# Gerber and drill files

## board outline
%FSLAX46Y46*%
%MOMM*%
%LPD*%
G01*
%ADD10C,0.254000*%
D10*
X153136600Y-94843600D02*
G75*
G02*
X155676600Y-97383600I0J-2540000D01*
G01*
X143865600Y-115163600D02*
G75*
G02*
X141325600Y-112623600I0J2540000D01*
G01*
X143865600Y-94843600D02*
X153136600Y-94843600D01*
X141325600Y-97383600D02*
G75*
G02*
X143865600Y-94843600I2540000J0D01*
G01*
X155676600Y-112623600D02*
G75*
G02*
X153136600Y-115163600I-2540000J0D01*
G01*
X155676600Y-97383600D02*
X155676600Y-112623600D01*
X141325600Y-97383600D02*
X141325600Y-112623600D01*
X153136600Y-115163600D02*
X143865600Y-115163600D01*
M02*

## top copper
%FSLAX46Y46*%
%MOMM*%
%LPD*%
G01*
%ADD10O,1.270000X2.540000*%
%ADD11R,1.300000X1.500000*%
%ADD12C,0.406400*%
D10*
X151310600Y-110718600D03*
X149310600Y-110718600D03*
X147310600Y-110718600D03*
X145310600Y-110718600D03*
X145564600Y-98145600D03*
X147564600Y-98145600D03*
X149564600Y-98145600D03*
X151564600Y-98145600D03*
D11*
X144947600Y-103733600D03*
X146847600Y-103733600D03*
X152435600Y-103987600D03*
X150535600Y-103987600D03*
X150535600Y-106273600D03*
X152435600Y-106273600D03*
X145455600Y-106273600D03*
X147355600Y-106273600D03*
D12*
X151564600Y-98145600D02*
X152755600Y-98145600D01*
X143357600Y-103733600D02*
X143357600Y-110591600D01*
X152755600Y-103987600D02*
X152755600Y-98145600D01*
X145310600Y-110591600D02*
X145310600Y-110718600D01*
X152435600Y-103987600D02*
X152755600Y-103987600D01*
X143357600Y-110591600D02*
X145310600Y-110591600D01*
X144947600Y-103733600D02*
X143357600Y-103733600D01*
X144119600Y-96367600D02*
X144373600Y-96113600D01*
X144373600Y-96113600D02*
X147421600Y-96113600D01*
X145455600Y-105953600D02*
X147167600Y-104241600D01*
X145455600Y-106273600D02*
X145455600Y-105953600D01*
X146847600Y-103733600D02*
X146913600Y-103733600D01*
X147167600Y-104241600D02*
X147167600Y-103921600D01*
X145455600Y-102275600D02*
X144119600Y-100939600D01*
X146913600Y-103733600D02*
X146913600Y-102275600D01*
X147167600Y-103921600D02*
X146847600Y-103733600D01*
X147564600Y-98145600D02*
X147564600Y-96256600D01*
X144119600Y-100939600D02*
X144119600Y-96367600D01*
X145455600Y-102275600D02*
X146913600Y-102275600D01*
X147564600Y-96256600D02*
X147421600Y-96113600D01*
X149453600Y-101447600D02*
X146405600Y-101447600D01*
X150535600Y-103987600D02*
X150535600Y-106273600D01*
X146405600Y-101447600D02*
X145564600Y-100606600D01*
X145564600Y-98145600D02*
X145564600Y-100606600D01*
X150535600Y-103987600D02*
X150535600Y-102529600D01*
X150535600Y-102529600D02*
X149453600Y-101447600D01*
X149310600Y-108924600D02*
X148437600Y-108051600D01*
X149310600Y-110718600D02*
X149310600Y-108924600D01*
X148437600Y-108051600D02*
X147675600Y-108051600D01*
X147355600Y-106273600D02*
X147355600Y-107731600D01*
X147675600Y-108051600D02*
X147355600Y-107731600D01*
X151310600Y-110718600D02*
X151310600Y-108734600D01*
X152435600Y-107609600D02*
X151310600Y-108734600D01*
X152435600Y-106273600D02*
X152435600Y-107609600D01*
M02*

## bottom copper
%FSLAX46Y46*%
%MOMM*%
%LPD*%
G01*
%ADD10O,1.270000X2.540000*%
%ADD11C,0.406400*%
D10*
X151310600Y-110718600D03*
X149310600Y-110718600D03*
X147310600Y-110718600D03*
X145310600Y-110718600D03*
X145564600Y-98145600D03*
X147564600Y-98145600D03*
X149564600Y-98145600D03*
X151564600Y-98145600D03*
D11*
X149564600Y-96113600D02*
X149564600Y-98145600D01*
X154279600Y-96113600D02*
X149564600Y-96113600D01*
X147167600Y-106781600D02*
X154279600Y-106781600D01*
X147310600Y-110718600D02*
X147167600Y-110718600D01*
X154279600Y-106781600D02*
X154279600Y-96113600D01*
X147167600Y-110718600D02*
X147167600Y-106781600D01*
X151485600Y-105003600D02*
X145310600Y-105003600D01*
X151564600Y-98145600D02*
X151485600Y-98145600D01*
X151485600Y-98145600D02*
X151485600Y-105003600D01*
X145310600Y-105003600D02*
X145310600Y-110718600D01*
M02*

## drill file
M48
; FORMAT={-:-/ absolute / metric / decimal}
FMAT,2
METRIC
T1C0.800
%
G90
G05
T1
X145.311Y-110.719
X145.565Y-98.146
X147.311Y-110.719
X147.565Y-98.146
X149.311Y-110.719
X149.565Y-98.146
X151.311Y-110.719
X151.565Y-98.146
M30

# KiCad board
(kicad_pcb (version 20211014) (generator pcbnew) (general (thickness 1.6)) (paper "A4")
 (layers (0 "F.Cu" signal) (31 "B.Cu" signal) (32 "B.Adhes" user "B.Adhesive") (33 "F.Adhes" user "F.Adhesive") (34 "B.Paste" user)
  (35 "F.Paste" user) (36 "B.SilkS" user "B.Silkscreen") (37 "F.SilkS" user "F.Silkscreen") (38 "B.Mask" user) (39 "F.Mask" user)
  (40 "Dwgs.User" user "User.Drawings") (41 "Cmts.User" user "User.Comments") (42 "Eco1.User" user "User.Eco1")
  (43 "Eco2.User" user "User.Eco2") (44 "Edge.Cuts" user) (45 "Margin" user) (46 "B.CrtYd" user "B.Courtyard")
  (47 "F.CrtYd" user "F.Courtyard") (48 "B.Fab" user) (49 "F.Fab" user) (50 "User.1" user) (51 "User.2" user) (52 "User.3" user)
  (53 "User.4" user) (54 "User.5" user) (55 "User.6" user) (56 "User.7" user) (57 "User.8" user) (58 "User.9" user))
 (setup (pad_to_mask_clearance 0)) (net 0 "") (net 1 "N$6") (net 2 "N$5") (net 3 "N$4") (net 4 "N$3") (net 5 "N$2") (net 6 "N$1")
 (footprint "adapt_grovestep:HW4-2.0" (layer "F.Cu") (at 148.3106 110.7186 180)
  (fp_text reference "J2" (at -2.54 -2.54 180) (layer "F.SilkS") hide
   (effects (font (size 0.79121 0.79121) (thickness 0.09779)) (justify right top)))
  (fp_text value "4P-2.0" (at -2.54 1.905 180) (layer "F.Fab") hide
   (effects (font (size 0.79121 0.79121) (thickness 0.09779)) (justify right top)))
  (pad "1" thru_hole oval (at -3 0 270) (size 2.54 1.27) (drill 0.8) (layers *.Cu *.Mask) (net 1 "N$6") (solder_mask_margin 0.1016))
  (pad "2" thru_hole oval (at -1 0 270) (size 2.54 1.27) (drill 0.8) (layers *.Cu *.Mask) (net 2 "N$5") (solder_mask_margin 0.1016))
  (pad "3" thru_hole oval (at 1 0 270) (size 2.54 1.27) (drill 0.8) (layers *.Cu *.Mask) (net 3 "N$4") (solder_mask_margin 0.1016))
  (pad "4" thru_hole oval (at 3 0 270) (size 2.54 1.27) (drill 0.8) (layers *.Cu *.Mask) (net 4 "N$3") (solder_mask_margin 0.1016)))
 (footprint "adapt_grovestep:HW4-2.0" (layer "F.Cu") (at 148.5646 98.1456)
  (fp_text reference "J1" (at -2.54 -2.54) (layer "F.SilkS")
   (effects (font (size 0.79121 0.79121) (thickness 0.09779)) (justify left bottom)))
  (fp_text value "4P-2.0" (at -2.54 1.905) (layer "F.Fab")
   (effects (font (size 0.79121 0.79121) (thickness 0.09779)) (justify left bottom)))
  (pad "1" thru_hole oval (at -3 0 90) (size 2.54 1.27) (drill 0.8) (layers *.Cu *.Mask) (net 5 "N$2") (solder_mask_margin 0.1016))
  (pad "2" thru_hole oval (at -1 0 90) (size 2.54 1.27) (drill 0.8) (layers *.Cu *.Mask) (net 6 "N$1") (solder_mask_margin 0.1016))
  (pad "3" thru_hole oval (at 1 0 90) (size 2.54 1.27) (drill 0.8) (layers *.Cu *.Mask) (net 3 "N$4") (solder_mask_margin 0.1016))
  (pad "4" thru_hole oval (at 3 0 90) (size 2.54 1.27) (drill 0.8) (layers *.Cu *.Mask) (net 4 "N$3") (solder_mask_margin 0.1016)))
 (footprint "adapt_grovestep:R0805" (layer "F.Cu") (at 145.8976 103.7336)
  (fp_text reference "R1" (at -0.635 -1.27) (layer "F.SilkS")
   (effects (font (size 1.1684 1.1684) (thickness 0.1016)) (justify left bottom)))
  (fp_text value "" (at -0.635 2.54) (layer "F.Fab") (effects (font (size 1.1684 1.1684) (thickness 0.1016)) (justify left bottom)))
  (pad "1" smd rect (at -0.95 0) (size 1.3 1.5) (layers "F.Cu" "F.Paste" "F.Mask") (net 4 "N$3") (solder_mask_margin 0.1016))
  (pad "2" smd rect (at 0.95 0) (size 1.3 1.5) (layers "F.Cu" "F.Paste" "F.Mask") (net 6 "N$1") (solder_mask_margin 0.1016)))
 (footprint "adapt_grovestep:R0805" (layer "F.Cu") (at 151.4856 103.9876 180)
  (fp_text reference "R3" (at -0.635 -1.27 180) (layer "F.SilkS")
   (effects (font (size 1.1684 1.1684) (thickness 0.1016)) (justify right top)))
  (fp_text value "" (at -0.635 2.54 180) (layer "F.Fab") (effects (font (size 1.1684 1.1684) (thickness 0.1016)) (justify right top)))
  (pad "1" smd rect (at -0.95 0 180) (size 1.3 1.5) (layers "F.Cu" "F.Paste" "F.Mask") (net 4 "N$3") (solder_mask_margin 0.1016))
  (pad "2" smd rect (at 0.95 0 180) (size 1.3 1.5) (layers "F.Cu" "F.Paste" "F.Mask") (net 5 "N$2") (solder_mask_margin 0.1016)))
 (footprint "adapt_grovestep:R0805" (layer "F.Cu") (at 151.4856 106.2736)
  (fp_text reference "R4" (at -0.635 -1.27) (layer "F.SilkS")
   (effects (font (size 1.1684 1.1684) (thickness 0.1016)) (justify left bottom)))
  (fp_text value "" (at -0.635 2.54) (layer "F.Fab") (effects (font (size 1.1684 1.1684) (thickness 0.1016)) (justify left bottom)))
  (pad "1" smd rect (at -0.95 0) (size 1.3 1.5) (layers "F.Cu" "F.Paste" "F.Mask") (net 5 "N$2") (solder_mask_margin 0.1016))
  (pad "2" smd rect (at 0.95 0) (size 1.3 1.5) (layers "F.Cu" "F.Paste" "F.Mask") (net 1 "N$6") (solder_mask_margin 0.1016)))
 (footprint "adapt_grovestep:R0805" (layer "F.Cu") (at 146.4056 106.2736)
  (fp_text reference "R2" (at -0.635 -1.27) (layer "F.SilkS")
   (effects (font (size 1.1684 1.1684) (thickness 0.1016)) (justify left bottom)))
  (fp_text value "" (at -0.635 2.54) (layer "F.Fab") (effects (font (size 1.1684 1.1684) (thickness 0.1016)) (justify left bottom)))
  (pad "1" smd rect (at -0.95 0) (size 1.3 1.5) (layers "F.Cu" "F.Paste" "F.Mask") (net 6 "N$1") (solder_mask_margin 0.1016))
  (pad "2" smd rect (at 0.95 0) (size 1.3 1.5) (layers "F.Cu" "F.Paste" "F.Mask") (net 2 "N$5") (solder_mask_margin 0.1016)))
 (gr_arc (start 153.1366 94.8436) (mid 154.932651 95.587549) (end 155.6766 97.3836) (layer "Edge.Cuts") (width 0.254))
 (gr_arc (start 143.8656 115.1636) (mid 142.069549 114.419651) (end 141.3256 112.6236) (layer "Edge.Cuts") (width 0.254))
 (gr_line (start 143.8656 94.8436) (end 153.1366 94.8436) (layer "Edge.Cuts") (width 0.254))
 (gr_arc (start 141.3256 97.3836) (mid 142.069549 95.587549) (end 143.8656 94.8436) (layer "Edge.Cuts") (width 0.254))
 (gr_arc (start 155.6766 112.6236) (mid 154.932651 114.419651) (end 153.1366 115.1636) (layer "Edge.Cuts") (width 0.254))
 (gr_line (start 155.6766 97.3836) (end 155.6766 112.6236) (layer "Edge.Cuts") (width 0.254))
 (gr_line (start 141.3256 97.3836) (end 141.3256 112.6236) (layer "Edge.Cuts") (width 0.254))
 (gr_line (start 153.1366 115.1636) (end 143.8656 115.1636) (layer "Edge.Cuts") (width 0.254))
 (segment (start 149.5646 96.1136) (end 149.5646 98.1456) (width 0.4064) (layer "B.Cu") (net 3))
 (segment (start 154.2796 96.1136) (end 149.5646 96.1136) (width 0.4064) (layer "B.Cu") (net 3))
 (segment (start 147.1676 106.7816) (end 154.2796 106.7816) (width 0.4064) (layer "B.Cu") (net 3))
 (segment (start 147.3106 110.7186) (end 147.1676 110.7186) (width 0.4064) (layer "B.Cu") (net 3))
 (segment (start 154.2796 106.7816) (end 154.2796 96.1136) (width 0.4064) (layer "B.Cu") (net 3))
 (segment (start 147.1676 110.7186) (end 147.1676 106.7816) (width 0.4064) (layer "B.Cu") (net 3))
 (segment (start 151.5646 98.1456) (end 152.7556 98.1456) (width 0.4064) (layer "F.Cu") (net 4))
 (segment (start 143.3576 103.7336) (end 143.3576 110.5916) (width 0.4064) (layer "F.Cu") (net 4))
 (segment (start 152.7556 103.9876) (end 152.7556 98.1456) (width 0.4064) (layer "F.Cu") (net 4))
 (segment (start 145.3106 110.5916) (end 145.3106 110.7186) (width 0.4064) (layer "F.Cu") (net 4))
 (segment (start 152.4356 103.9876) (end 152.7556 103.9876) (width 0.4064) (layer "F.Cu") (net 4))
 (segment (start 143.3576 110.5916) (end 145.3106 110.5916) (width 0.4064) (layer "F.Cu") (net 4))
 (segment (start 144.9476 103.7336) (end 143.3576 103.7336) (width 0.4064) (layer "F.Cu") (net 4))
 (segment (start 151.4856 105.0036) (end 145.3106 105.0036) (width 0.4064) (layer "B.Cu") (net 4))
 (segment (start 151.5646 98.1456) (end 151.4856 98.1456) (width 0.4064) (layer "B.Cu") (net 4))
 (segment (start 151.4856 98.1456) (end 151.4856 105.0036) (width 0.4064) (layer "B.Cu") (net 4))
 (segment (start 145.3106 105.0036) (end 145.3106 110.7186) (width 0.4064) (layer "B.Cu") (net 4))
 (segment (start 144.1196 96.3676) (end 144.3736 96.1136) (width 0.4064) (layer "F.Cu") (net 6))
 (segment (start 144.3736 96.1136) (end 147.4216 96.1136) (width 0.4064) (layer "F.Cu") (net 6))
 (segment (start 145.4556 105.9536) (end 147.1676 104.2416) (width 0.4064) (layer "F.Cu") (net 6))
 (segment (start 145.4556 106.2736) (end 145.4556 105.9536) (width 0.4064) (layer "F.Cu") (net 6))
 (segment (start 146.8476 103.7336) (end 146.9136 103.7336) (width 0.4064) (layer "F.Cu") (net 6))
 (segment (start 147.1676 104.2416) (end 147.1676 103.9216) (width 0.4064) (layer "F.Cu") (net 6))
 (segment (start 145.4556 102.2756) (end 144.1196 100.9396) (width 0.4064) (layer "F.Cu") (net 6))
 (segment (start 146.9136 103.7336) (end 146.9136 102.2756) (width 0.4064) (layer "F.Cu") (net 6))
 (segment (start 147.1676 103.9216) (end 146.8476 103.7336) (width 0.4064) (layer "F.Cu") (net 6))
 (segment (start 147.5646 98.1456) (end 147.5646 96.2566) (width 0.4064) (layer "F.Cu") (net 6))
 (segment (start 144.1196 100.9396) (end 144.1196 96.3676) (width 0.4064) (layer "F.Cu") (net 6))
 (segment (start 145.4556 102.2756) (end 146.9136 102.2756) (width 0.4064) (layer "F.Cu") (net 6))
 (segment (start 147.5646 96.2566) (end 147.4216 96.1136) (width 0.4064) (layer "F.Cu") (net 6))
 (segment (start 149.4536 101.4476) (end 146.4056 101.4476) (width 0.4064) (layer "F.Cu") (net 5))
 (segment (start 150.5356 103.9876) (end 150.5356 106.2736) (width 0.4064) (layer "F.Cu") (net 5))
 (segment (start 146.4056 101.4476) (end 145.5646 100.6066) (width 0.4064) (layer "F.Cu") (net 5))
 (segment (start 145.5646 98.1456) (end 145.5646 100.6066) (width 0.4064) (layer "F.Cu") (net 5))
 (segment (start 150.5356 103.9876) (end 150.5356 102.5296) (width 0.4064) (layer "F.Cu") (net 5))
 (segment (start 150.5356 102.5296) (end 149.4536 101.4476) (width 0.4064) (layer "F.Cu") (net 5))
 (segment (start 149.3106 108.9246) (end 148.4376 108.0516) (width 0.4064) (layer "F.Cu") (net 2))
 (segment (start 149.3106 110.7186) (end 149.3106 108.9246) (width 0.4064) (layer "F.Cu") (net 2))
 (segment (start 148.4376 108.0516) (end 147.6756 108.0516) (width 0.4064) (layer "F.Cu") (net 2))
 (segment (start 147.3556 106.2736) (end 147.3556 107.7316) (width 0.4064) (layer "F.Cu") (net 2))
 (segment (start 147.6756 108.0516) (end 147.3556 107.7316) (width 0.4064) (layer "F.Cu") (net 2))
 (segment (start 151.3106 110.7186) (end 151.3106 108.7346) (width 0.4064) (layer "F.Cu") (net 1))
 (segment (start 152.4356 107.6096) (end 151.3106 108.7346) (width 0.4064) (layer "F.Cu") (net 1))
 (segment (start 152.4356 106.2736) (end 152.4356 107.6096) (width 0.4064) (layer "F.Cu") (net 1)))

